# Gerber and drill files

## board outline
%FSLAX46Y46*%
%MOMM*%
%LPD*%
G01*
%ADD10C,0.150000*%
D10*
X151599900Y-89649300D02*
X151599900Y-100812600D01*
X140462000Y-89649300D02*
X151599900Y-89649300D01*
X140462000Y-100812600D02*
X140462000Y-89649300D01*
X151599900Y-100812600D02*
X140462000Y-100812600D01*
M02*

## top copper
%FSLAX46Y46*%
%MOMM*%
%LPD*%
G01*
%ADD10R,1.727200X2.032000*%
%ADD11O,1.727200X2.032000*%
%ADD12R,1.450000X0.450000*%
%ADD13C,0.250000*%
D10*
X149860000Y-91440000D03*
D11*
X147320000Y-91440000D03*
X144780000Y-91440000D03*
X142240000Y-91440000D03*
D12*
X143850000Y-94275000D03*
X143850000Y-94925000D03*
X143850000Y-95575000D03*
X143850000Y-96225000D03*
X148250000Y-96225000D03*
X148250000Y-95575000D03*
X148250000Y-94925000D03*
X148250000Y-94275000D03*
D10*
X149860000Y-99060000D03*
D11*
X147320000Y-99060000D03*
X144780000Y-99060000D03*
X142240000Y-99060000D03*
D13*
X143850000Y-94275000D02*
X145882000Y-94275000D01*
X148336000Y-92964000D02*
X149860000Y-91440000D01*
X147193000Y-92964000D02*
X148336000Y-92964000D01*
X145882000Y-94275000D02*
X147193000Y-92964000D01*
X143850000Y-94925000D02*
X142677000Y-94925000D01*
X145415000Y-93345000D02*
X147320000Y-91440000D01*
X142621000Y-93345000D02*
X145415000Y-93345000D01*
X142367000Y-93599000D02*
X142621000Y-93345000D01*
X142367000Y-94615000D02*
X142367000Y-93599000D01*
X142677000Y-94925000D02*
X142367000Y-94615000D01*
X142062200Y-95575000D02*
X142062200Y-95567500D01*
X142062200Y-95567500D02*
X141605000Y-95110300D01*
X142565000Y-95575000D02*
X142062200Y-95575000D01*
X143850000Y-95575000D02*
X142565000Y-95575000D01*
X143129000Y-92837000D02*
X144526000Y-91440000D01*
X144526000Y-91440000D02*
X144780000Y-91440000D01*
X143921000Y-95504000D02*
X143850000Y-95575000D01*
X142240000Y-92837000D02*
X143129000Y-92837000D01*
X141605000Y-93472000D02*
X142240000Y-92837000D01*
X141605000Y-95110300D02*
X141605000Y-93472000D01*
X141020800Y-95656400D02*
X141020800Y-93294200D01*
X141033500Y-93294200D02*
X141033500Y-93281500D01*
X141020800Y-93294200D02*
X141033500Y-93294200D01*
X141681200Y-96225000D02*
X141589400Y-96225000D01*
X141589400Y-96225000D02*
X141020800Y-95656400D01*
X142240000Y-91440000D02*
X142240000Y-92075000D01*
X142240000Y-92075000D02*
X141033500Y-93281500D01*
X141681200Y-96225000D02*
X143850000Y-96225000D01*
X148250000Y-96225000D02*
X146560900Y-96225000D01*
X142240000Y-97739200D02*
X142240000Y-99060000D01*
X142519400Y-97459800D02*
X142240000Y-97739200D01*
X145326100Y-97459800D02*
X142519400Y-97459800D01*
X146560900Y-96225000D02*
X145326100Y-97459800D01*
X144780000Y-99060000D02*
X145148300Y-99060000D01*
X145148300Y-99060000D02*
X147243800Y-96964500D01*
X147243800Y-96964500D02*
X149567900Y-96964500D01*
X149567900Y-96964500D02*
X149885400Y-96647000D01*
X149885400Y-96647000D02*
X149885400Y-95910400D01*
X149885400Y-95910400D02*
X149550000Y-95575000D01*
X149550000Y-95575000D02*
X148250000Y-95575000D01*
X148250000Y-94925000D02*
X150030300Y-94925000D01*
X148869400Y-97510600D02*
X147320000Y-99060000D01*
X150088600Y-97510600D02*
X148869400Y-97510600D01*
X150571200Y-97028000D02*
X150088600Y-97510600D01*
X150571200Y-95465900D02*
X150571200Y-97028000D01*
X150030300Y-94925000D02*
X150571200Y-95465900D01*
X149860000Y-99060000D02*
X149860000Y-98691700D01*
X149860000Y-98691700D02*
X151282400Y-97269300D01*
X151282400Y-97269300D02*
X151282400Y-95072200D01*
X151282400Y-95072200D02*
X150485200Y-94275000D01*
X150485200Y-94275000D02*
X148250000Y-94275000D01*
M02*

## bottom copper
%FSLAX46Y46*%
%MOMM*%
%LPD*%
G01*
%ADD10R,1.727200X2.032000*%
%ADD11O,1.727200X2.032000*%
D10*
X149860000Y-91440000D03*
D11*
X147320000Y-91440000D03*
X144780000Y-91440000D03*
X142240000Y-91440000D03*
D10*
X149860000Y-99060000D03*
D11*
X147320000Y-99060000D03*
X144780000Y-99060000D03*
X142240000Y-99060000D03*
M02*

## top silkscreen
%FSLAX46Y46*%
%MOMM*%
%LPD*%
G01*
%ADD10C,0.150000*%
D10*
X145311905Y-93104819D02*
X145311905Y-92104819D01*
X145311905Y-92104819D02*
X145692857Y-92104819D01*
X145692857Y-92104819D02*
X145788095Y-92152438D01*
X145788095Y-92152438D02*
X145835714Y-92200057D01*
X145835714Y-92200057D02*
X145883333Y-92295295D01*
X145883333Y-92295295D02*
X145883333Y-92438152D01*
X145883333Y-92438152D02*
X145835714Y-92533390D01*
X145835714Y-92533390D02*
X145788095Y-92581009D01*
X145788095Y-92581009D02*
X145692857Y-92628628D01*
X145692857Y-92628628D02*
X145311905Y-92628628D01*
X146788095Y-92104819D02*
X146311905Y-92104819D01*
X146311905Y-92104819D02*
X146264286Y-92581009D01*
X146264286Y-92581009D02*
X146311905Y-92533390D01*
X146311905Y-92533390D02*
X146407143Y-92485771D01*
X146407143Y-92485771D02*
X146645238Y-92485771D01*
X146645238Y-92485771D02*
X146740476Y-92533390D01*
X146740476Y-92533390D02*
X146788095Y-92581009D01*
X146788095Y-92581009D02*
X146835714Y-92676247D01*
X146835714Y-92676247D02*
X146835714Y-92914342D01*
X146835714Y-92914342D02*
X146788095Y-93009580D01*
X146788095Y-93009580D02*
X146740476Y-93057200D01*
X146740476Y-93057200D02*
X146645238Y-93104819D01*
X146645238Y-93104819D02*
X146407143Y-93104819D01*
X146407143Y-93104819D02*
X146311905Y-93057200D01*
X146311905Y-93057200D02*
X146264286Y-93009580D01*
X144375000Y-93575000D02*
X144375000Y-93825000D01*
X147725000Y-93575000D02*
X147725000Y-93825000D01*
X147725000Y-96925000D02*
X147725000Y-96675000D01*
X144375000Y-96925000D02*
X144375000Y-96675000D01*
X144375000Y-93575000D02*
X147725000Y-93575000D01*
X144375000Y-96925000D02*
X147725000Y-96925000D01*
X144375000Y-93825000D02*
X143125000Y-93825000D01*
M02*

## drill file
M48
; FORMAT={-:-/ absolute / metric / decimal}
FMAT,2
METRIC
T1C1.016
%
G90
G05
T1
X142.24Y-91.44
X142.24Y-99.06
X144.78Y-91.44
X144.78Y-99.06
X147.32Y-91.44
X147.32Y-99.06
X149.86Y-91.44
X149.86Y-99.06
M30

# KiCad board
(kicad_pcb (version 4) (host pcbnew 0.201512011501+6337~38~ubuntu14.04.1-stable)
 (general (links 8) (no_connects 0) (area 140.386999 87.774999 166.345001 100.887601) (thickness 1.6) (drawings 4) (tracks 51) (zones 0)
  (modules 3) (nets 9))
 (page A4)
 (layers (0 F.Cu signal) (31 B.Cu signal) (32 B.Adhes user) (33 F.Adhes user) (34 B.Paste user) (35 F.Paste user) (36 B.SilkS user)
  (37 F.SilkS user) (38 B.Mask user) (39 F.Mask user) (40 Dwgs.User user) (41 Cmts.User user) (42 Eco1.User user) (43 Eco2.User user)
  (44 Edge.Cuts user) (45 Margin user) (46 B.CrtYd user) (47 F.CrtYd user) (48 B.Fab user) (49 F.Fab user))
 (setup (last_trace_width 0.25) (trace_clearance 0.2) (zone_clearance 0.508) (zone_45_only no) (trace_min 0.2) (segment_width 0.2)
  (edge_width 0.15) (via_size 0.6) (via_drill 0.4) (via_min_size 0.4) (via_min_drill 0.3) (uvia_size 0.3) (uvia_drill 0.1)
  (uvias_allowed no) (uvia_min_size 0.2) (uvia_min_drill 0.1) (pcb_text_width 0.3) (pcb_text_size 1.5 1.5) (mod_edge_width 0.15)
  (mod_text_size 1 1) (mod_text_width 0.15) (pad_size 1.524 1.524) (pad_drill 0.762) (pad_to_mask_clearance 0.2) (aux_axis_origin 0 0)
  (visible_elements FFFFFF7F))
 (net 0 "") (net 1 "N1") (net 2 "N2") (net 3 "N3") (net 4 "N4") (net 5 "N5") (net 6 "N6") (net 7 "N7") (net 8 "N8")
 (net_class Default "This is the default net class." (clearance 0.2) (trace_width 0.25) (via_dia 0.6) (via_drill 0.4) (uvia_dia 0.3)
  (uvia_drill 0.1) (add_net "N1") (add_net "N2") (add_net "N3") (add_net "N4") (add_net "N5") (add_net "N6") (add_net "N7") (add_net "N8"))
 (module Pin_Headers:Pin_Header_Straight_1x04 (layer B.Cu) (at 149.86 91.44 90)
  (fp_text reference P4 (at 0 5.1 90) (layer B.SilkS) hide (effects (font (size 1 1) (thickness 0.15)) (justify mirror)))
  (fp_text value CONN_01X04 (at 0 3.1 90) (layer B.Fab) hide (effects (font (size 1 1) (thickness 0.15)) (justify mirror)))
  (pad 1 thru_hole rect (at 0 0 90) (size 2.032 1.7272) (drill 1.016) (layers *.Cu *.Mask B.SilkS) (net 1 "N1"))
  (pad 2 thru_hole oval (at 0 -2.54 90) (size 2.032 1.7272) (drill 1.016) (layers *.Cu *.Mask B.SilkS) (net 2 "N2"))
  (pad 3 thru_hole oval (at 0 -5.08 90) (size 2.032 1.7272) (drill 1.016) (layers *.Cu *.Mask B.SilkS) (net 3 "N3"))
  (pad 4 thru_hole oval (at 0 -7.62 90) (size 2.032 1.7272) (drill 1.016) (layers *.Cu *.Mask B.SilkS) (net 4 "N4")))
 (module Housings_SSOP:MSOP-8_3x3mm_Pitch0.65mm (layer F.Cu) (at 146.05 95.25)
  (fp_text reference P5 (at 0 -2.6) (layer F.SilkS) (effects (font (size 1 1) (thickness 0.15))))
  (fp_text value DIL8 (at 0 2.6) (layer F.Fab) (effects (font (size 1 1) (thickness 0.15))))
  (fp_line (start -1.675 -1.675) (end -1.675 -1.425) (layer F.SilkS) (width 0.15))
  (fp_line (start 1.675 -1.675) (end 1.675 -1.425) (layer F.SilkS) (width 0.15))
  (fp_line (start 1.675 1.675) (end 1.675 1.425) (layer F.SilkS) (width 0.15))
  (fp_line (start -1.675 1.675) (end -1.675 1.425) (layer F.SilkS) (width 0.15))
  (fp_line (start -1.675 -1.675) (end 1.675 -1.675) (layer F.SilkS) (width 0.15))
  (fp_line (start -1.675 1.675) (end 1.675 1.675) (layer F.SilkS) (width 0.15))
  (fp_line (start -1.675 -1.425) (end -2.925 -1.425) (layer F.SilkS) (width 0.15))
  (pad 1 smd rect (at -2.2 -0.975) (size 1.45 0.45) (layers F.Cu F.Paste F.Mask) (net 1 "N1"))
  (pad 2 smd rect (at -2.2 -0.325) (size 1.45 0.45) (layers F.Cu F.Paste F.Mask) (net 2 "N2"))
  (pad 3 smd rect (at -2.2 0.325) (size 1.45 0.45) (layers F.Cu F.Paste F.Mask) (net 3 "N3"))
  (pad 4 smd rect (at -2.2 0.975) (size 1.45 0.45) (layers F.Cu F.Paste F.Mask) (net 4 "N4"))
  (pad 5 smd rect (at 2.2 0.975) (size 1.45 0.45) (layers F.Cu F.Paste F.Mask) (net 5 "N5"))
  (pad 6 smd rect (at 2.2 0.325) (size 1.45 0.45) (layers F.Cu F.Paste F.Mask) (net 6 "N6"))
  (pad 7 smd rect (at 2.2 -0.325) (size 1.45 0.45) (layers F.Cu F.Paste F.Mask) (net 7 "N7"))
  (pad 8 smd rect (at 2.2 -0.975) (size 1.45 0.45) (layers F.Cu F.Paste F.Mask) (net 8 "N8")))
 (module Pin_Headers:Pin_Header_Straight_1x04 (layer B.Cu) (at 149.86 99.06 90)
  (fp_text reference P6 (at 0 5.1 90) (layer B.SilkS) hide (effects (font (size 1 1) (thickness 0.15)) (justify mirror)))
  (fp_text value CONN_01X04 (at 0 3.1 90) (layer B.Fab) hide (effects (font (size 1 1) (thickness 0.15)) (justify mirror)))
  (pad 1 thru_hole rect (at 0 0 90) (size 2.032 1.7272) (drill 1.016) (layers *.Cu *.Mask B.SilkS) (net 8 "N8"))
  (pad 2 thru_hole oval (at 0 -2.54 90) (size 2.032 1.7272) (drill 1.016) (layers *.Cu *.Mask B.SilkS) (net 7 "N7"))
  (pad 3 thru_hole oval (at 0 -5.08 90) (size 2.032 1.7272) (drill 1.016) (layers *.Cu *.Mask B.SilkS) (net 6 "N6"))
  (pad 4 thru_hole oval (at 0 -7.62 90) (size 2.032 1.7272) (drill 1.016) (layers *.Cu *.Mask B.SilkS) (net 5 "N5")))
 (gr_line (start 151.5999 89.6493) (end 151.5999 100.8126) (angle 90) (layer Edge.Cuts) (width 0.15))
 (gr_line (start 140.462 89.6493) (end 151.5999 89.6493) (angle 90) (layer Edge.Cuts) (width 0.15))
 (gr_line (start 140.462 100.8126) (end 140.462 89.6493) (angle 90) (layer Edge.Cuts) (width 0.15))
 (gr_line (start 151.5999 100.8126) (end 140.462 100.8126) (angle 90) (layer Edge.Cuts) (width 0.15))
 (segment (start 143.85 94.275) (end 145.882 94.275) (width 0.25) (layer F.Cu) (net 1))
 (segment (start 148.336 92.964) (end 149.86 91.44) (width 0.25) (layer F.Cu) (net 1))
 (segment (start 147.193 92.964) (end 148.336 92.964) (width 0.25) (layer F.Cu) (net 1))
 (segment (start 145.882 94.275) (end 147.193 92.964) (width 0.25) (layer F.Cu) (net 1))
 (segment (start 143.85 94.925) (end 142.677 94.925) (width 0.25) (layer F.Cu) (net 2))
 (segment (start 145.415 93.345) (end 147.32 91.44) (width 0.25) (layer F.Cu) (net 2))
 (segment (start 142.621 93.345) (end 145.415 93.345) (width 0.25) (layer F.Cu) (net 2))
 (segment (start 142.367 93.599) (end 142.621 93.345) (width 0.25) (layer F.Cu) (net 2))
 (segment (start 142.367 94.615) (end 142.367 93.599) (width 0.25) (layer F.Cu) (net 2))
 (segment (start 142.677 94.925) (end 142.367 94.615) (width 0.25) (layer F.Cu) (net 2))
 (segment (start 142.0622 95.575) (end 142.0622 95.5675) (width 0.25) (layer F.Cu) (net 3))
 (segment (start 142.0622 95.5675) (end 141.605 95.1103) (width 0.25) (layer F.Cu) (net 3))
 (segment (start 142.565 95.575) (end 142.0622 95.575) (width 0.25) (layer F.Cu) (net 3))
 (segment (start 143.85 95.575) (end 142.565 95.575) (width 0.25) (layer F.Cu) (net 3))
 (segment (start 143.129 92.837) (end 144.526 91.44) (width 0.25) (layer F.Cu) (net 3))
 (segment (start 144.526 91.44) (end 144.78 91.44) (width 0.25) (layer F.Cu) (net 3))
 (segment (start 143.921 95.504) (end 143.85 95.575) (width 0.25) (layer F.Cu) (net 3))
 (segment (start 142.24 92.837) (end 143.129 92.837) (width 0.25) (layer F.Cu) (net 3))
 (segment (start 141.605 93.472) (end 142.24 92.837) (width 0.25) (layer F.Cu) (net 3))
 (segment (start 141.605 95.1103) (end 141.605 93.472) (width 0.25) (layer F.Cu) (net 3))
 (segment (start 141.0208 95.6564) (end 141.0208 93.2942) (width 0.25) (layer F.Cu) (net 4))
 (segment (start 141.0335 93.2942) (end 141.0335 93.2815) (width 0.25) (layer F.Cu) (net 4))
 (segment (start 141.0208 93.2942) (end 141.0335 93.2942) (width 0.25) (layer F.Cu) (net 4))
 (segment (start 141.6812 96.225) (end 141.5894 96.225) (width 0.25) (layer F.Cu) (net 4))
 (segment (start 141.5894 96.225) (end 141.0208 95.6564) (width 0.25) (layer F.Cu) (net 4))
 (segment (start 142.24 91.44) (end 142.24 92.075) (width 0.25) (layer F.Cu) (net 4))
 (segment (start 142.24 92.075) (end 141.0335 93.2815) (width 0.25) (layer F.Cu) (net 4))
 (segment (start 141.6812 96.225) (end 143.85 96.225) (width 0.25) (layer F.Cu) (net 4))
 (segment (start 148.25 96.225) (end 146.5609 96.225) (width 0.25) (layer F.Cu) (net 5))
 (segment (start 142.24 97.7392) (end 142.24 99.06) (width 0.25) (layer F.Cu) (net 5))
 (segment (start 142.5194 97.4598) (end 142.24 97.7392) (width 0.25) (layer F.Cu) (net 5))
 (segment (start 145.3261 97.4598) (end 142.5194 97.4598) (width 0.25) (layer F.Cu) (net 5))
 (segment (start 146.5609 96.225) (end 145.3261 97.4598) (width 0.25) (layer F.Cu) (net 5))
 (segment (start 144.78 99.06) (end 145.1483 99.06) (width 0.25) (layer F.Cu) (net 6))
 (segment (start 145.1483 99.06) (end 147.2438 96.9645) (width 0.25) (layer F.Cu) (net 6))
 (segment (start 147.2438 96.9645) (end 149.5679 96.9645) (width 0.25) (layer F.Cu) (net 6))
 (segment (start 149.5679 96.9645) (end 149.8854 96.647) (width 0.25) (layer F.Cu) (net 6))
 (segment (start 149.8854 96.647) (end 149.8854 95.9104) (width 0.25) (layer F.Cu) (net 6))
 (segment (start 149.8854 95.9104) (end 149.55 95.575) (width 0.25) (layer F.Cu) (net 6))
 (segment (start 149.55 95.575) (end 148.25 95.575) (width 0.25) (layer F.Cu) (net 6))
 (segment (start 148.25 94.925) (end 150.0303 94.925) (width 0.25) (layer F.Cu) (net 7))
 (segment (start 148.8694 97.5106) (end 147.32 99.06) (width 0.25) (layer F.Cu) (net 7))
 (segment (start 150.0886 97.5106) (end 148.8694 97.5106) (width 0.25) (layer F.Cu) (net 7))
 (segment (start 150.5712 97.028) (end 150.0886 97.5106) (width 0.25) (layer F.Cu) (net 7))
 (segment (start 150.5712 95.4659) (end 150.5712 97.028) (width 0.25) (layer F.Cu) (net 7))
 (segment (start 150.0303 94.925) (end 150.5712 95.4659) (width 0.25) (layer F.Cu) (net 7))
 (segment (start 149.86 99.06) (end 149.86 98.6917) (width 0.25) (layer F.Cu) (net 8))
 (segment (start 149.86 98.6917) (end 151.2824 97.2693) (width 0.25) (layer F.Cu) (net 8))
 (segment (start 151.2824 97.2693) (end 151.2824 95.0722) (width 0.25) (layer F.Cu) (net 8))
 (segment (start 151.2824 95.0722) (end 150.4852 94.275) (width 0.25) (layer F.Cu) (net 8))
 (segment (start 150.4852 94.275) (end 148.25 94.275) (width 0.25) (layer F.Cu) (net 8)))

